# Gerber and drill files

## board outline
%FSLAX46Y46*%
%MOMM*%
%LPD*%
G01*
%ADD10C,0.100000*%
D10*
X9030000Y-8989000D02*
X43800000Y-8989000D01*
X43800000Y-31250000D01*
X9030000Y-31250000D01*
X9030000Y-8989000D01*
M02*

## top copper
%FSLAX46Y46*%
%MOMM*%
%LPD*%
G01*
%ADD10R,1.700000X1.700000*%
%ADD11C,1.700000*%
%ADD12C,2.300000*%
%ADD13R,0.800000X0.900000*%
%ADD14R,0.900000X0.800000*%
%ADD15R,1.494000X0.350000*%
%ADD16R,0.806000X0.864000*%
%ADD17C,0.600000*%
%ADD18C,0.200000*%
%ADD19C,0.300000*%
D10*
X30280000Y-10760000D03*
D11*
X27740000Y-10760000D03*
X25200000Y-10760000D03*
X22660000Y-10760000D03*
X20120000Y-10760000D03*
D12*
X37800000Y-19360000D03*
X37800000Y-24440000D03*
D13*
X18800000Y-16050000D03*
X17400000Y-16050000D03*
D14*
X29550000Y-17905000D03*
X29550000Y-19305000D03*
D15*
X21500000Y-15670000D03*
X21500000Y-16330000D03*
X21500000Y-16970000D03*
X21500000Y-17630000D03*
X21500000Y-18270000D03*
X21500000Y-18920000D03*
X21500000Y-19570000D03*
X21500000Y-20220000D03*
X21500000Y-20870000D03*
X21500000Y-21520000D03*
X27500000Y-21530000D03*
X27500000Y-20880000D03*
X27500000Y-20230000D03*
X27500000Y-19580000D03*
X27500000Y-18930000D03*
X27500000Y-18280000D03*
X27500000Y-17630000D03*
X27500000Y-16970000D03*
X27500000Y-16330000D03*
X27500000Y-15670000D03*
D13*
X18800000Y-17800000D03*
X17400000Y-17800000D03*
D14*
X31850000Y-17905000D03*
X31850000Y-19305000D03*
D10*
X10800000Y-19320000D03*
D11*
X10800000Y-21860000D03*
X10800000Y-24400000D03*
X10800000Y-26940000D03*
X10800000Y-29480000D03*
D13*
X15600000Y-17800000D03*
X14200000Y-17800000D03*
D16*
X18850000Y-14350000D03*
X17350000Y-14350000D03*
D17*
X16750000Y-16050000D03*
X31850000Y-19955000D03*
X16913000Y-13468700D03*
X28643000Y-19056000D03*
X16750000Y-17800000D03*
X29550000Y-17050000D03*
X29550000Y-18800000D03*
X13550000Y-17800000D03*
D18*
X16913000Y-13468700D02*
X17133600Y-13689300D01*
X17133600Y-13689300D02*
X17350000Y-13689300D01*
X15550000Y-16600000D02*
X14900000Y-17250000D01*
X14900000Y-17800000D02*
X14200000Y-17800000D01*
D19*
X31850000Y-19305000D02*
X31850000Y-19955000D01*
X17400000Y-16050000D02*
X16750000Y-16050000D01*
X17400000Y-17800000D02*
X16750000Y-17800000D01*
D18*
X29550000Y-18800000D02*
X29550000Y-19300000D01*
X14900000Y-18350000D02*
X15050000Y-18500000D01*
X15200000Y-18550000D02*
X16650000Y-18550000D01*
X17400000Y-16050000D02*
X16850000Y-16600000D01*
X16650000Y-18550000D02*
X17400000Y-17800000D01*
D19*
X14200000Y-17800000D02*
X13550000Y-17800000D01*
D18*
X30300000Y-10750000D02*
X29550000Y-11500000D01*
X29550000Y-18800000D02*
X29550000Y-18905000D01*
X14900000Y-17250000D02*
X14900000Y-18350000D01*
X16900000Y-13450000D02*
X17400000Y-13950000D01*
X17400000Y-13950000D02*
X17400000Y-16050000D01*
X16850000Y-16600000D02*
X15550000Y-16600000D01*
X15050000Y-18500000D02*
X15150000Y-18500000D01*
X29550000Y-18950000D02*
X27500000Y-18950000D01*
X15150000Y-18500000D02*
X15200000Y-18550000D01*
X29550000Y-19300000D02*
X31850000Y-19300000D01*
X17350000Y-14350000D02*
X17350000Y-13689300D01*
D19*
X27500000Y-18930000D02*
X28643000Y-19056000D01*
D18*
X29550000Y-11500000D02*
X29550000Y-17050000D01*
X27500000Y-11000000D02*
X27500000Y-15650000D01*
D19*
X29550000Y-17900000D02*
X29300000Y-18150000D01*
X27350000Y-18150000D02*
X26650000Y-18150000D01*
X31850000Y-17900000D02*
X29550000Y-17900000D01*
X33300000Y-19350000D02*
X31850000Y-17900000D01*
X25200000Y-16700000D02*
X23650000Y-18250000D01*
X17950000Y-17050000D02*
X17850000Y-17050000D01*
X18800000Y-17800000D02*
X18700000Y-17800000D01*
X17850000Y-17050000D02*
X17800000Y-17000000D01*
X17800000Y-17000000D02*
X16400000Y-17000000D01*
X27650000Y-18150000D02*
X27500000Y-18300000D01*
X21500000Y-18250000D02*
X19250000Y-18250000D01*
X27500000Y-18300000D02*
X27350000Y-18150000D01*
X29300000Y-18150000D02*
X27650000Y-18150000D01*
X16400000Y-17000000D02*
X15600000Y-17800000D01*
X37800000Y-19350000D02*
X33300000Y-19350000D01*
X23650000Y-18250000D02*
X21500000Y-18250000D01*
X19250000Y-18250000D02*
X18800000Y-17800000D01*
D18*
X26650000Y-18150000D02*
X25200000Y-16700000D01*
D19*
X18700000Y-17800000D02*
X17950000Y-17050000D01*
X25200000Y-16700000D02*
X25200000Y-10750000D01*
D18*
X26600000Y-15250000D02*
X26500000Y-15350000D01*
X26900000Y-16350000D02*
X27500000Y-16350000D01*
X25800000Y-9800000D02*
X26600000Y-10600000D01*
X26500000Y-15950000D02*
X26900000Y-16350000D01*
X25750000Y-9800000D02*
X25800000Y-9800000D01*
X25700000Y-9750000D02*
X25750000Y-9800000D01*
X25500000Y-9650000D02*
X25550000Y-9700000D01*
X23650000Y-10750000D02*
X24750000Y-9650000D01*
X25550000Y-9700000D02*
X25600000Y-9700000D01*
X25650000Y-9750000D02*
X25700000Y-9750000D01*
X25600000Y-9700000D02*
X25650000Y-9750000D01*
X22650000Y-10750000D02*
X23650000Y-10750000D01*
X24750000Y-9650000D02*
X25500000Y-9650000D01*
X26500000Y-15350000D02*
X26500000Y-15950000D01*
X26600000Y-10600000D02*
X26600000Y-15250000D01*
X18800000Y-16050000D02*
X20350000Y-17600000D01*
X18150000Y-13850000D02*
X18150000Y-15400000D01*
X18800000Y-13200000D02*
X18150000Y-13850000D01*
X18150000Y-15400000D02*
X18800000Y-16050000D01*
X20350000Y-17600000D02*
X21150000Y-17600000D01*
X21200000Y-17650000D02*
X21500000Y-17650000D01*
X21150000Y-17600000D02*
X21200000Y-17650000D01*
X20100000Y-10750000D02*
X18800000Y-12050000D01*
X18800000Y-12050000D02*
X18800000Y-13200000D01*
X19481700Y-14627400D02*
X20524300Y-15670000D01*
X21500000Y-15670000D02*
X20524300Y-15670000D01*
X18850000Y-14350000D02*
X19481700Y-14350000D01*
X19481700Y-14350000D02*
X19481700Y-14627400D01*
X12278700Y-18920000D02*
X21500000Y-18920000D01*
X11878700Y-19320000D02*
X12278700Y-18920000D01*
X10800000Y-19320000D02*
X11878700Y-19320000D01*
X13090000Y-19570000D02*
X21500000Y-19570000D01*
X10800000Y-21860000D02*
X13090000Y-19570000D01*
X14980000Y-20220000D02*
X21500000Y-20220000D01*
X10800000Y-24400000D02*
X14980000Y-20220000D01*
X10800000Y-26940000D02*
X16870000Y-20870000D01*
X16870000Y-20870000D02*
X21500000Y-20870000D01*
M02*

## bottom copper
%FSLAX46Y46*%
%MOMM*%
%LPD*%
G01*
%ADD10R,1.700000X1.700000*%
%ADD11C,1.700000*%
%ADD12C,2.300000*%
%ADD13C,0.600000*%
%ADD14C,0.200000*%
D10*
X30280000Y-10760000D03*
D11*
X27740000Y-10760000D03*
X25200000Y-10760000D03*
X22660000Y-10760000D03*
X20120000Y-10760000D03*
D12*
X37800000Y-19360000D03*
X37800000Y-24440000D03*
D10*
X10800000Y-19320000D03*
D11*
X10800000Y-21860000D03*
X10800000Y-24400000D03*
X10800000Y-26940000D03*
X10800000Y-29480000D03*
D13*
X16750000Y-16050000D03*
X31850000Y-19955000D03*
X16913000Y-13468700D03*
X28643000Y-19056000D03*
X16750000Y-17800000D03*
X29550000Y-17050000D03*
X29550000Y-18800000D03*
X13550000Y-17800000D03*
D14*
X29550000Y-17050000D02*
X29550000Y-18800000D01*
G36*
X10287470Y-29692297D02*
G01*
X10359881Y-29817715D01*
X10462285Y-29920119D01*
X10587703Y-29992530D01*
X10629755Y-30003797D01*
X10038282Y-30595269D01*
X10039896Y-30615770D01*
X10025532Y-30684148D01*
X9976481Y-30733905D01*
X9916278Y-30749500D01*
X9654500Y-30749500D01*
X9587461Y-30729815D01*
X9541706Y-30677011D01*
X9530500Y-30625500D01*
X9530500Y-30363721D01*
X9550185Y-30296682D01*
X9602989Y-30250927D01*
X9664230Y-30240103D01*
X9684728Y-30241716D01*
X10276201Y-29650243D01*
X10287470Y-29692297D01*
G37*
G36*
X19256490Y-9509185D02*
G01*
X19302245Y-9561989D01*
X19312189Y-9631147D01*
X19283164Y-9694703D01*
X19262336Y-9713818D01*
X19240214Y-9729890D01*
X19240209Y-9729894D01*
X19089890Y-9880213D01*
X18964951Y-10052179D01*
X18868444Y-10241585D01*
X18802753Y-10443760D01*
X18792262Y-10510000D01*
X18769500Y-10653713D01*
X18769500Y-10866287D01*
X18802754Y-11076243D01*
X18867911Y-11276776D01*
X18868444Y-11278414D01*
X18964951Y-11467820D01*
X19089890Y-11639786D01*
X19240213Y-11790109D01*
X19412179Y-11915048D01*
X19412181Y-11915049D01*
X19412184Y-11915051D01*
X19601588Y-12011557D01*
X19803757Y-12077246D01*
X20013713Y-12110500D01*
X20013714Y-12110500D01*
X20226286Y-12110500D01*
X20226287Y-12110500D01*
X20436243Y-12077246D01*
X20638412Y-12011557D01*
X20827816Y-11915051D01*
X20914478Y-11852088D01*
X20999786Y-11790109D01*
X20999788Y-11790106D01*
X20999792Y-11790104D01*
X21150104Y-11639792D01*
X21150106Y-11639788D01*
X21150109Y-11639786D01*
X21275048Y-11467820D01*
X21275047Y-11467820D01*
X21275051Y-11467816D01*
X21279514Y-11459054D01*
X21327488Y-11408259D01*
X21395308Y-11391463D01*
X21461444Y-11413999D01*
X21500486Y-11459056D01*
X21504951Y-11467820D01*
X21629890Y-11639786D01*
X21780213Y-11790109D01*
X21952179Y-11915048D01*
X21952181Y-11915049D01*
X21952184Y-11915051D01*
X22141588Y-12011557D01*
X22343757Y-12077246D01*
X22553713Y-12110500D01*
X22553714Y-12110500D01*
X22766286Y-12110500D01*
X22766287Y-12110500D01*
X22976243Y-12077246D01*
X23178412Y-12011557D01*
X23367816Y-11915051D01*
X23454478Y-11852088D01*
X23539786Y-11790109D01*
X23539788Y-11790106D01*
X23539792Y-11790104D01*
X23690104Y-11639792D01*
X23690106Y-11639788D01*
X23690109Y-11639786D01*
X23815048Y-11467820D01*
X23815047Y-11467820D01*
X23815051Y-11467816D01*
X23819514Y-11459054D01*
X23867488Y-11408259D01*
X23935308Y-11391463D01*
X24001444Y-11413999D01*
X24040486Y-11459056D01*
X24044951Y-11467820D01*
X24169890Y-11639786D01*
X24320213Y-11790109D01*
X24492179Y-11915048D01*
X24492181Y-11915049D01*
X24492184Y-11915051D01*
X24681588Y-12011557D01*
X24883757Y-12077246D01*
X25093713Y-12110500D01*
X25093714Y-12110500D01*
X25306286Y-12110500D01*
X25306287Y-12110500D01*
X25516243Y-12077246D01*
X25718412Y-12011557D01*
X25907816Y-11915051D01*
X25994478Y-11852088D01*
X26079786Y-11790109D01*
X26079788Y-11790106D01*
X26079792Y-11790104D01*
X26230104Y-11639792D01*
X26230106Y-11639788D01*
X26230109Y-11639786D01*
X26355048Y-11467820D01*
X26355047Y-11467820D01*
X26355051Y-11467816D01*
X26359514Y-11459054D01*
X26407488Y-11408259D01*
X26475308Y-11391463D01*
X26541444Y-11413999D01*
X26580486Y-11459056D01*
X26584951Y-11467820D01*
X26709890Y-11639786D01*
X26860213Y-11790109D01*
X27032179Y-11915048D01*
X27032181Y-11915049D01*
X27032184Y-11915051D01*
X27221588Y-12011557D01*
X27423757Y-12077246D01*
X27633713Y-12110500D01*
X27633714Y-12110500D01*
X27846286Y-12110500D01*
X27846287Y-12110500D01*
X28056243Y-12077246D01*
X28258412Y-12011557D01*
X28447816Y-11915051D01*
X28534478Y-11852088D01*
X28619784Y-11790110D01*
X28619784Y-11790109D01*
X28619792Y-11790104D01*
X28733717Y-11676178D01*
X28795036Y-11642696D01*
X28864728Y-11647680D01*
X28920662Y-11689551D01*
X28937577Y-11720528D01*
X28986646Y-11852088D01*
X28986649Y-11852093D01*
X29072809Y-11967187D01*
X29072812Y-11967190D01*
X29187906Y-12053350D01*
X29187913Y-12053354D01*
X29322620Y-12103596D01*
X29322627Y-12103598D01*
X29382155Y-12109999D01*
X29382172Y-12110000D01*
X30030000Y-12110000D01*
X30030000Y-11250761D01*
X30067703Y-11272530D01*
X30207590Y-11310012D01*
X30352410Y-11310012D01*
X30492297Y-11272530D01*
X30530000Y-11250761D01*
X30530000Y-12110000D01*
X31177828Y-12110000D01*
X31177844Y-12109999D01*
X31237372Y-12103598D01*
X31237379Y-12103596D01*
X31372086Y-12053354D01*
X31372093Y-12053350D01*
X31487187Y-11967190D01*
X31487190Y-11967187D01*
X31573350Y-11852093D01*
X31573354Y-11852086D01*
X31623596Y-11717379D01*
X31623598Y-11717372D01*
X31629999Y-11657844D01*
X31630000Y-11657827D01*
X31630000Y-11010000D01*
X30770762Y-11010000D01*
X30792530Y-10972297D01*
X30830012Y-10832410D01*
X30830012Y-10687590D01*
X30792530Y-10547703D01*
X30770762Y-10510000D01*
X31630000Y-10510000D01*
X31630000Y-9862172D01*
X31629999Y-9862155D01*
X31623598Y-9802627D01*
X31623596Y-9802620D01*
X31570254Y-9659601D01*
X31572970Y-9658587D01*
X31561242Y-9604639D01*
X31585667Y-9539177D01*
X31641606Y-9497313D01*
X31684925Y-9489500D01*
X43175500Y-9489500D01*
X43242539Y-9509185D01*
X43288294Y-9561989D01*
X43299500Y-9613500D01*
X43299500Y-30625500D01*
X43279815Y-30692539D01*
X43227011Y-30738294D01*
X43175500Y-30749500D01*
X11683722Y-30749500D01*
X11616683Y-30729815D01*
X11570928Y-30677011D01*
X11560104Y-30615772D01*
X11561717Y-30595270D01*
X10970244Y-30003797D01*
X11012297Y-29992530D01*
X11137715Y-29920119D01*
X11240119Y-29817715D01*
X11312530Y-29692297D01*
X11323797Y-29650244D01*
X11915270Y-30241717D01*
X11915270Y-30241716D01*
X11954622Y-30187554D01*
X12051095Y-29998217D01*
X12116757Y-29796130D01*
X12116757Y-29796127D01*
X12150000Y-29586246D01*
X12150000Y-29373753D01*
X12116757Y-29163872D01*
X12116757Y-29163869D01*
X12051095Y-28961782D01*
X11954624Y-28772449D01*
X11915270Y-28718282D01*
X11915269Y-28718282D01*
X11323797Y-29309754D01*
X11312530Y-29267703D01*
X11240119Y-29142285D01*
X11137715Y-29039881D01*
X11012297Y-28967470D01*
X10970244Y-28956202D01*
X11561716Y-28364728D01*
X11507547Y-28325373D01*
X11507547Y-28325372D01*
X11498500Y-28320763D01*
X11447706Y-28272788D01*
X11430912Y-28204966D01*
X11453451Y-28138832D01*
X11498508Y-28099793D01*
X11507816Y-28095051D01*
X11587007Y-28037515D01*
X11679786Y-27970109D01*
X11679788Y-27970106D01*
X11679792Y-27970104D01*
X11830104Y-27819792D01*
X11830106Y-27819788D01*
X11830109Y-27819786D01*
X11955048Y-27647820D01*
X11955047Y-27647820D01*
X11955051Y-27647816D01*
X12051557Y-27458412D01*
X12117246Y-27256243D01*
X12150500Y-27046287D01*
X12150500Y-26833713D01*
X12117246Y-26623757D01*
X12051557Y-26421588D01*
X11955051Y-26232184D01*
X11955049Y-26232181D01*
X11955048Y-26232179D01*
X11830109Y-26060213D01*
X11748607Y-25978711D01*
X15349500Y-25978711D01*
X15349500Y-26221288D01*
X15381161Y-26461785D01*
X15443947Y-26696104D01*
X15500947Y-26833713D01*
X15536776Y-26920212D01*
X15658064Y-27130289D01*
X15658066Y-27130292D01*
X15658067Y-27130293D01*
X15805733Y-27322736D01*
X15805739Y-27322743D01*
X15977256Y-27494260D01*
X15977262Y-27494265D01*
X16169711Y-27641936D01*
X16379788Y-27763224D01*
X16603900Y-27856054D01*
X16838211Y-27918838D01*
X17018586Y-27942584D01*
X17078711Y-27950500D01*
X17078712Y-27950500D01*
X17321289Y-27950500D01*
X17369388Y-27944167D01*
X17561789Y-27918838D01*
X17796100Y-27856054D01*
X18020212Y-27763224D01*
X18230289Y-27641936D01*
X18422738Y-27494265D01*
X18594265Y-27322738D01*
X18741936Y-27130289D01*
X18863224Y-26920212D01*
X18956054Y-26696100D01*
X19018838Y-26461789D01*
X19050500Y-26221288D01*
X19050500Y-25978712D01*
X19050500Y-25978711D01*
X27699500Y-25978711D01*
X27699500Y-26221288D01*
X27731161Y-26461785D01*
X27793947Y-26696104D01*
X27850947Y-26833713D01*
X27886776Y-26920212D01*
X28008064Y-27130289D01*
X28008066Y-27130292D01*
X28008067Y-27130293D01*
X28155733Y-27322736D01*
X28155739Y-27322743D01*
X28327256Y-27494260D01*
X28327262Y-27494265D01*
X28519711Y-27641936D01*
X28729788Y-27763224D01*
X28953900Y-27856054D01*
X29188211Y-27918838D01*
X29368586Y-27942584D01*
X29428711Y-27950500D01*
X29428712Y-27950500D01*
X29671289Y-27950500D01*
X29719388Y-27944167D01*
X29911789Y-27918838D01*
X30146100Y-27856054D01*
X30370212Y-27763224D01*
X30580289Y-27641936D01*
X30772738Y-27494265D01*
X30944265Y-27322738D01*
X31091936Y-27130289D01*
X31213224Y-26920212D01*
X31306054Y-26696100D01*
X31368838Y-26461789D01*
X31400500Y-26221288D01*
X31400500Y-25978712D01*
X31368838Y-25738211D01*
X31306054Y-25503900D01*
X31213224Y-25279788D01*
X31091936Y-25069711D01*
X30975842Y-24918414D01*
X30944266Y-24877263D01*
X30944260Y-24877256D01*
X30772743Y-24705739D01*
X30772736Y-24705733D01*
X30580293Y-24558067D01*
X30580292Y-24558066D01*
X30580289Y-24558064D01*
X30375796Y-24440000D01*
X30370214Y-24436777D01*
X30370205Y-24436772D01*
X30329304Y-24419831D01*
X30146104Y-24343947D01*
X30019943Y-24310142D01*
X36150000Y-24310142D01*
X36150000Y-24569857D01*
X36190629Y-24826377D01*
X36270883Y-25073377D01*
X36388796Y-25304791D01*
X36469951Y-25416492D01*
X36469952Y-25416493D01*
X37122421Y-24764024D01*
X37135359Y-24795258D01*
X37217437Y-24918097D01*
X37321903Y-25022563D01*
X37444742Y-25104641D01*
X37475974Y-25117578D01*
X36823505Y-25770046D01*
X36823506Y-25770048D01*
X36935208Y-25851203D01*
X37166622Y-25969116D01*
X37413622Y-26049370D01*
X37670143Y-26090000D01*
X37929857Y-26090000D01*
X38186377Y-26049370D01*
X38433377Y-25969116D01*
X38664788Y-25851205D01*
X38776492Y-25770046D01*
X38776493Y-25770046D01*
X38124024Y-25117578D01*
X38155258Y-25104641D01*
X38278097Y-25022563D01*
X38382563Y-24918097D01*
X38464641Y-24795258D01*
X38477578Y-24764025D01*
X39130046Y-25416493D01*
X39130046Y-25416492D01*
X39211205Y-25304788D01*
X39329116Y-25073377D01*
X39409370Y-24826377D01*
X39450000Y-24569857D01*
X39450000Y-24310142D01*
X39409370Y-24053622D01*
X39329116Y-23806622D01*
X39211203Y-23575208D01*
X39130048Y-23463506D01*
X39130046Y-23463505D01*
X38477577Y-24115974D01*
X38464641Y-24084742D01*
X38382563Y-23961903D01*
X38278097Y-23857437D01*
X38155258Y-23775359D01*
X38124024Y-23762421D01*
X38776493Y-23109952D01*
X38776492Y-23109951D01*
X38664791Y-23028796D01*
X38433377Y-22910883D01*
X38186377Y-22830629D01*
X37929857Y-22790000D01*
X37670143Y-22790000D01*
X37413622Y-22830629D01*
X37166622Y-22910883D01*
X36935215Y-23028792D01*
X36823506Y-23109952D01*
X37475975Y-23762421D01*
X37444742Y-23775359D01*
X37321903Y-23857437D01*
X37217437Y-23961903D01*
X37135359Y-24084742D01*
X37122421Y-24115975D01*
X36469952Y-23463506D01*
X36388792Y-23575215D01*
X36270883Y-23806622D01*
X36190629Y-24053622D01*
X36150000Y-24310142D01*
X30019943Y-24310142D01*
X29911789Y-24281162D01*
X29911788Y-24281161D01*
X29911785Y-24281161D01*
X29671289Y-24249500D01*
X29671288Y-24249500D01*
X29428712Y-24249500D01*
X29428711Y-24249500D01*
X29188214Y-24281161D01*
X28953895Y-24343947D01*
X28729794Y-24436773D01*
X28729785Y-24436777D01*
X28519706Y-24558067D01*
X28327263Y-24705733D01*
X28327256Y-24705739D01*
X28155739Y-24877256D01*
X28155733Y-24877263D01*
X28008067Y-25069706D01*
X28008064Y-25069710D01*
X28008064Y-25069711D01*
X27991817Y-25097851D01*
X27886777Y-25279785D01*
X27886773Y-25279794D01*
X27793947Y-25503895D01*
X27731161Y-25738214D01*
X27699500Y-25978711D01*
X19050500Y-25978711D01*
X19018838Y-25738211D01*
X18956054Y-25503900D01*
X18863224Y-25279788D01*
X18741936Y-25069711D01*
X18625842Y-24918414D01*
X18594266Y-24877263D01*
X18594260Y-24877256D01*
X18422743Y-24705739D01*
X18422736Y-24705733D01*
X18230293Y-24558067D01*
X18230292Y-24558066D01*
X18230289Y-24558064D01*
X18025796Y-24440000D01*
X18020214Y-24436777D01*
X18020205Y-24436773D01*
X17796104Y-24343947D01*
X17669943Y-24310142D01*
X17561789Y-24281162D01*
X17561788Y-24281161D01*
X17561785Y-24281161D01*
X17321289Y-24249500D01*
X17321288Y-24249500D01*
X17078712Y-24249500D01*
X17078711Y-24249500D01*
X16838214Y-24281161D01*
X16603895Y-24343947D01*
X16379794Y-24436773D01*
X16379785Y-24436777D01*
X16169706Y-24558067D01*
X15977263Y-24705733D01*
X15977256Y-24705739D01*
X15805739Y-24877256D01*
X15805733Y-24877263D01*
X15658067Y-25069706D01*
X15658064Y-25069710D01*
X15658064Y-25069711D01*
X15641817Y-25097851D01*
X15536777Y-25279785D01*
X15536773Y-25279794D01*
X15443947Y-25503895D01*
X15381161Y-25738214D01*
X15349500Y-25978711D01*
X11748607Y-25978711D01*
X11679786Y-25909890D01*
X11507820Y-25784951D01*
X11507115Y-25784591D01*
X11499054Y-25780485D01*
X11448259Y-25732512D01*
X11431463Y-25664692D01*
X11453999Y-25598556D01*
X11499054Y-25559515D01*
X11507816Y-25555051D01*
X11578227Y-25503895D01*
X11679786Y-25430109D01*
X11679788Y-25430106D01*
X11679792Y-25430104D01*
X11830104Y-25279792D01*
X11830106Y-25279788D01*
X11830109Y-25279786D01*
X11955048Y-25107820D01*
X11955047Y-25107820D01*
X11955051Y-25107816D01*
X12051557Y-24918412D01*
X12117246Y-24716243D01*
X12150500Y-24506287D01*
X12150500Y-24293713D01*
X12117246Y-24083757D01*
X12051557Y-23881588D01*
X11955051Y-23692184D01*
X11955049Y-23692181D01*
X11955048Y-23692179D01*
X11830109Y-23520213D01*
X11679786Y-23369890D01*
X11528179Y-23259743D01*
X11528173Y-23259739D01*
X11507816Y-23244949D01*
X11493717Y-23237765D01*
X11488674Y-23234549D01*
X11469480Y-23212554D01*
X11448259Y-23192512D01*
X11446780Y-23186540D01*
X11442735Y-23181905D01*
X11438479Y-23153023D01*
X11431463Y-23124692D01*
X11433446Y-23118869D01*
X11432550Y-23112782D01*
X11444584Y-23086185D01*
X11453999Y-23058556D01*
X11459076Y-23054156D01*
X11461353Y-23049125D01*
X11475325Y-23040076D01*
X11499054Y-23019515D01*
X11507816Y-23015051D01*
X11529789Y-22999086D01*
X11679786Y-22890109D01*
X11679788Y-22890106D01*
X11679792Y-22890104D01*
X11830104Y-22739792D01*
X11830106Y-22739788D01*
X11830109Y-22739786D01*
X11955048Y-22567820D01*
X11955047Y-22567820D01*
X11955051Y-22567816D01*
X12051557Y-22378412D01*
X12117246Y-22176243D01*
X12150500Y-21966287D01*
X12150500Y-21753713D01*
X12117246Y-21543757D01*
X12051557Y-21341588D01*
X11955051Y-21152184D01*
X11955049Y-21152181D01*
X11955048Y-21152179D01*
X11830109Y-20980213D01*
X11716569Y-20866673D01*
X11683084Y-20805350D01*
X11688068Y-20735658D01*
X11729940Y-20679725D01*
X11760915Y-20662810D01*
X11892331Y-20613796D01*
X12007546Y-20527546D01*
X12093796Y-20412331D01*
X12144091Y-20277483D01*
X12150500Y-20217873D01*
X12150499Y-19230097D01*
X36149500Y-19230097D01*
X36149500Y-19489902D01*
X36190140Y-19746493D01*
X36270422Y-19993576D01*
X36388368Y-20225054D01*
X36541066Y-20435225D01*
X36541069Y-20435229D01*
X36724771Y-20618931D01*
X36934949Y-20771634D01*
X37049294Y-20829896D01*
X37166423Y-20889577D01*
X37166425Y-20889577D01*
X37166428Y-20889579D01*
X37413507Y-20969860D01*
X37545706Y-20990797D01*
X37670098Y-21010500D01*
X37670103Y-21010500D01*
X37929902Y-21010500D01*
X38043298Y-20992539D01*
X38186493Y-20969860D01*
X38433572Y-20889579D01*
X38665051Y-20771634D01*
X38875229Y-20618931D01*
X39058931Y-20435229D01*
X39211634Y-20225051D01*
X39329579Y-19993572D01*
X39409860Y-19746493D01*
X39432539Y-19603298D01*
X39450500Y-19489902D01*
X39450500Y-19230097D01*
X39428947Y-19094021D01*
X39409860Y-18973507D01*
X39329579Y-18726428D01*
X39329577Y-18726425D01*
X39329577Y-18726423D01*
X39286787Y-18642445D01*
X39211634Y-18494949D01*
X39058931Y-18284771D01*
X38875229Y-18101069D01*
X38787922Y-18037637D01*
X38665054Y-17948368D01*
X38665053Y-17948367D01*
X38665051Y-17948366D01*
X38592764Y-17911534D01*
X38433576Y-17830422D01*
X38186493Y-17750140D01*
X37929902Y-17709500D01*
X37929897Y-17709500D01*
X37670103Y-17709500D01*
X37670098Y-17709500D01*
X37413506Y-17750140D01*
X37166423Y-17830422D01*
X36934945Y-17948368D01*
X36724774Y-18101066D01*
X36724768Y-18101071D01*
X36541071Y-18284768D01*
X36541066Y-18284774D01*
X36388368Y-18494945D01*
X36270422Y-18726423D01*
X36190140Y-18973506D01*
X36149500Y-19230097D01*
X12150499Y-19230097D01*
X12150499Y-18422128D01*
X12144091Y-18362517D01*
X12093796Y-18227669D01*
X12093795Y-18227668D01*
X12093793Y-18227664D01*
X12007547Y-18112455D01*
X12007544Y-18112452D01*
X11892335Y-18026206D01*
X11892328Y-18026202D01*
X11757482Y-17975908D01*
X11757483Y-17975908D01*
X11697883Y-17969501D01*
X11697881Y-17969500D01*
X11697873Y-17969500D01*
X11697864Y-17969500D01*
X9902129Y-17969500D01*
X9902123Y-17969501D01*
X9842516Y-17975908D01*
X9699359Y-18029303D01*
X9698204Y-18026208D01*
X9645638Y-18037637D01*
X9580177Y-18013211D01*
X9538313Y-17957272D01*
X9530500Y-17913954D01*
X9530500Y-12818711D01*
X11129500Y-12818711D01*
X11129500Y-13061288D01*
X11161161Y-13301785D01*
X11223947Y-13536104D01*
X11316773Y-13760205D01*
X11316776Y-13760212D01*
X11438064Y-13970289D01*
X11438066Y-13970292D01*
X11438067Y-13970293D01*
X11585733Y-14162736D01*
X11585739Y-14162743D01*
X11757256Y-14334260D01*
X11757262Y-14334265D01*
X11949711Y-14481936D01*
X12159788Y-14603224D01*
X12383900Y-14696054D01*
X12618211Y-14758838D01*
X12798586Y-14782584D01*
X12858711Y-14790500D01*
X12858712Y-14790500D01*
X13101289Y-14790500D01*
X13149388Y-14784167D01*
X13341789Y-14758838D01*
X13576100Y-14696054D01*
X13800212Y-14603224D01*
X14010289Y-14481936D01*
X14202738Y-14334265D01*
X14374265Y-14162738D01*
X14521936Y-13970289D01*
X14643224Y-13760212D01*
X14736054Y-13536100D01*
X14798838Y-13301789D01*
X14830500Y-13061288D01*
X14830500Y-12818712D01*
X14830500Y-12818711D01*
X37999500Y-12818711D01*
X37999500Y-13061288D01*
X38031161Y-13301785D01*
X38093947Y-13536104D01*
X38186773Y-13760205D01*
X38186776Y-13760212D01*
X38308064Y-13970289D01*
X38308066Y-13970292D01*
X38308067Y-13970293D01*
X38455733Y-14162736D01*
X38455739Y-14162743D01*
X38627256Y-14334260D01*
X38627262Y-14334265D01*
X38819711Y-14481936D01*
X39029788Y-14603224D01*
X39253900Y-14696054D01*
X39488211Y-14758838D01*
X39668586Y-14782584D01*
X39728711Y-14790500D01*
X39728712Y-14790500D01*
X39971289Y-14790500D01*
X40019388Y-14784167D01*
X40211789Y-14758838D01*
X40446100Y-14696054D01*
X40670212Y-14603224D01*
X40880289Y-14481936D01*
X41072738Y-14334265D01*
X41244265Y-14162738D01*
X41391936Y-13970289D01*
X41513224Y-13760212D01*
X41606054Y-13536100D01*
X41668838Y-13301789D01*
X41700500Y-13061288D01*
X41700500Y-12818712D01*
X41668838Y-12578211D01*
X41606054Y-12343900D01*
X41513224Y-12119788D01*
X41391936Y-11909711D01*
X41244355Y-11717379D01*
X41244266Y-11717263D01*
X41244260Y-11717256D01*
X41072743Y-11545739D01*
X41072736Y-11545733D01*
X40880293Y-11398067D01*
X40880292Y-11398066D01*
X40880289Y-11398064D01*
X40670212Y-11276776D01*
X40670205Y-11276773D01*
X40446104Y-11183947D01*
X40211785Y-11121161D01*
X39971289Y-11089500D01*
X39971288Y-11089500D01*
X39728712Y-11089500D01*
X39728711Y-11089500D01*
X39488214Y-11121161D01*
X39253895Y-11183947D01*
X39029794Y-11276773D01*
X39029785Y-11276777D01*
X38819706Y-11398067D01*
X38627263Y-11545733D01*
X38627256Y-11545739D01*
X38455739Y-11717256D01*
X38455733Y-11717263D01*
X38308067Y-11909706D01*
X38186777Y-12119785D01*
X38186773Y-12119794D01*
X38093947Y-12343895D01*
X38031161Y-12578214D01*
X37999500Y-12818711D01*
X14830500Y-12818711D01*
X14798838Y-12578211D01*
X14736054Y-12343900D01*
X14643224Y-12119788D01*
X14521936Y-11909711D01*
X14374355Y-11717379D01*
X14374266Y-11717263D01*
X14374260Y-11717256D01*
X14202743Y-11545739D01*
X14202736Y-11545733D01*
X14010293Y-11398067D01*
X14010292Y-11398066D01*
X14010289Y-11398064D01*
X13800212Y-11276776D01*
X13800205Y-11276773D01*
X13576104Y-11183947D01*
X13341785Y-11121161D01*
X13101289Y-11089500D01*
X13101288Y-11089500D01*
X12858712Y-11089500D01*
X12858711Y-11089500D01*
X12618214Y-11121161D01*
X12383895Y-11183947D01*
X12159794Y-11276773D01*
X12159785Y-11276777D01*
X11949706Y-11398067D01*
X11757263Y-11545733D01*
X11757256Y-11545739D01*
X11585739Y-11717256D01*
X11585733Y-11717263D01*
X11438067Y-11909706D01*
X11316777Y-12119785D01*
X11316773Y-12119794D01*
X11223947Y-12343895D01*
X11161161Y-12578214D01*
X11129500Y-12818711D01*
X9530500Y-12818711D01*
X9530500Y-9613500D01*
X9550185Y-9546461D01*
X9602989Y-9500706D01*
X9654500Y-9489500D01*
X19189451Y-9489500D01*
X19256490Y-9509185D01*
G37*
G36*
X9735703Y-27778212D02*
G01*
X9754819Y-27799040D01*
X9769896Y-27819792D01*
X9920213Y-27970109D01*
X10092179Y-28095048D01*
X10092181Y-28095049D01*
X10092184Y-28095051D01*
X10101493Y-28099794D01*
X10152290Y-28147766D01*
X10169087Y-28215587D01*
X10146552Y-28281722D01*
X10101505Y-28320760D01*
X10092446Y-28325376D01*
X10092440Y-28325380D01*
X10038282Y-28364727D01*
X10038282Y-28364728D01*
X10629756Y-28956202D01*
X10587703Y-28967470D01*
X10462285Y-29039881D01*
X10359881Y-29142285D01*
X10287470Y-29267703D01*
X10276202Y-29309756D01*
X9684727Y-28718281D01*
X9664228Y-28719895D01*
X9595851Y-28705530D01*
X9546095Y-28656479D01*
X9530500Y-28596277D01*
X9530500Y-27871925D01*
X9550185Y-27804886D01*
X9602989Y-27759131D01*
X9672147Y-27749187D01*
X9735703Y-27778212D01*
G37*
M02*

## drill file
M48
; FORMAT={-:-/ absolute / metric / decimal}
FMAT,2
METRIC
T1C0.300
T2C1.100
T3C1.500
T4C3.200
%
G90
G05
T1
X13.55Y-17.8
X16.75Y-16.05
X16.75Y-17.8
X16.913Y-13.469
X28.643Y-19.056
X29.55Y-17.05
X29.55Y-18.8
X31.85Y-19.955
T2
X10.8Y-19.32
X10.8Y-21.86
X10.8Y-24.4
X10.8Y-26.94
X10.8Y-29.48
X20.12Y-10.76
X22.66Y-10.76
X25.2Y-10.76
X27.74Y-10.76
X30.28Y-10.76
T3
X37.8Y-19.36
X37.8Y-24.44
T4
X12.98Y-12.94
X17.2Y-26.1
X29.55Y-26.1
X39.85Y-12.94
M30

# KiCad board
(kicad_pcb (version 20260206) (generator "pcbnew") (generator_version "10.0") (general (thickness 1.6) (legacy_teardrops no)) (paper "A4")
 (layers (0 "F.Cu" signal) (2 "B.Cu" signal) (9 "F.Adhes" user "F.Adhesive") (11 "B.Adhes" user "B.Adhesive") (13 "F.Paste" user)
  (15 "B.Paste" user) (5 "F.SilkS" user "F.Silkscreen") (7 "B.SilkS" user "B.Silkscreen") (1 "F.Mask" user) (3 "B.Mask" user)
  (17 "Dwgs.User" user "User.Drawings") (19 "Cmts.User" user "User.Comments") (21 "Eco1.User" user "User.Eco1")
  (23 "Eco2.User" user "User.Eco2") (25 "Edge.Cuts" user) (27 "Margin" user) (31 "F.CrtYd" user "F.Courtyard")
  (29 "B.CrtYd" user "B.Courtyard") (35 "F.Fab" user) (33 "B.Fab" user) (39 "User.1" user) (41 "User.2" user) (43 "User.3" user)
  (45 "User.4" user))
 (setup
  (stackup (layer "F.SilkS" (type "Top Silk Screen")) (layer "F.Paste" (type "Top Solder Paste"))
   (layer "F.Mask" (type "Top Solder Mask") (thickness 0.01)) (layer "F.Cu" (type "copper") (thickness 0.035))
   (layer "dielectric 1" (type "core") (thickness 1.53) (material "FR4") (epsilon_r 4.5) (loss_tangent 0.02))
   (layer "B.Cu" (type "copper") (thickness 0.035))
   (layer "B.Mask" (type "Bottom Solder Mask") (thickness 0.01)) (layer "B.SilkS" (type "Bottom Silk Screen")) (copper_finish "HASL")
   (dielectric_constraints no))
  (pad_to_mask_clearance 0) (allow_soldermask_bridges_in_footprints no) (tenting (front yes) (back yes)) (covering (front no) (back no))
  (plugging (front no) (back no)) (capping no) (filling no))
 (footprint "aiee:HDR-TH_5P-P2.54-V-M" (layer "F.Cu") (at 25.2 10.76 180)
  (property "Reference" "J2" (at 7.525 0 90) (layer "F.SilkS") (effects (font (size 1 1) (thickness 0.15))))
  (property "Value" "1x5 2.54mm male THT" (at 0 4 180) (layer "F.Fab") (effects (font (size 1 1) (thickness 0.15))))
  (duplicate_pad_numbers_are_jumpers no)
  (pad "1" thru_hole rect (at -5.08 0 180) (size 1.7 1.7) (drill 1.100024) (layers "*.Cu" "*.Mask") (remove_unused_layers no) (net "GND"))
  (pad "2" thru_hole circle (at -2.54 0 180) (size 1.7 1.7) (drill 1.100024) (layers "*.Cu" "*.Mask") (remove_unused_layers no)
   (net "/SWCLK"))
  (pad "3" thru_hole circle (at 0 0 180) (size 1.7 1.7) (drill 1.100024) (layers "*.Cu" "*.Mask") (remove_unused_layers no) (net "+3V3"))
  (pad "4" thru_hole circle (at 2.54 0 180) (size 1.7 1.7) (drill 1.100024) (layers "*.Cu" "*.Mask") (remove_unused_layers no)
   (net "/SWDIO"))
  (pad "5" thru_hole circle (at 5.08 0 180) (size 1.7 1.7) (drill 1.100024) (layers "*.Cu" "*.Mask") (remove_unused_layers no) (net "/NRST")))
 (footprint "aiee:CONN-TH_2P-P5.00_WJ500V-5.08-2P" (layer "F.Cu") (at 37.8 21.9 -90)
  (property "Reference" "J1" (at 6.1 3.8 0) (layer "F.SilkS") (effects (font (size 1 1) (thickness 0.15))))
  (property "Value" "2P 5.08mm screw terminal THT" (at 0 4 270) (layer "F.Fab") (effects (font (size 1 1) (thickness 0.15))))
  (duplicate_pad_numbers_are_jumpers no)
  (pad "1" thru_hole circle (at -2.54 0 90) (size 2.3 2.3) (drill 1.5) (layers "*.Cu" "*.Mask") (remove_unused_layers no) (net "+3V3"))
  (pad "2" thru_hole circle (at 2.54 0 90) (size 2.3 2.3) (drill 1.5) (layers "*.Cu" "*.Mask") (remove_unused_layers no) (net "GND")))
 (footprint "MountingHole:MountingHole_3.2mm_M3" (layer "F.Cu") (at 29.55 26.1)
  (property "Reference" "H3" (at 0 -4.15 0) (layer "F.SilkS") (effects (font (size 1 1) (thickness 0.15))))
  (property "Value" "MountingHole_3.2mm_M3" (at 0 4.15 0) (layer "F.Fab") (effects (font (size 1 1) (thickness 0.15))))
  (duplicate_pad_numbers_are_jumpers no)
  (pad "" np_thru_hole circle (at 0 0) (size 3.2 3.2) (drill 3.2) (layers "*.Cu" "*.Mask")))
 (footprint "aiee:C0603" (layer "F.Cu") (at 18.1 16.05 180)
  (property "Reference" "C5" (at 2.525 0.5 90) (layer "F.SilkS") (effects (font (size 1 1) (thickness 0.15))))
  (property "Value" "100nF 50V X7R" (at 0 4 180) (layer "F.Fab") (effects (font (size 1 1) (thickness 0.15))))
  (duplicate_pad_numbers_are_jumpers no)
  (pad "1" smd rect (at -0.7 0 180) (size 0.8 0.9) (layers "F.Cu" "F.Mask" "F.Paste") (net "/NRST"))
  (pad "2" smd rect (at 0.7 0 180) (size 0.8 0.9) (layers "F.Cu" "F.Mask" "F.Paste") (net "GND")))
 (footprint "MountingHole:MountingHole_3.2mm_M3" (layer "F.Cu") (at 17.2 26.1)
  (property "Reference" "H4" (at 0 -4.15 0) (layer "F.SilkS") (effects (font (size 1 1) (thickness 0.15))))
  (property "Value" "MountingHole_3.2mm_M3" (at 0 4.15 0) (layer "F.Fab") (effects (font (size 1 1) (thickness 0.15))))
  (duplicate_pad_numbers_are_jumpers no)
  (pad "" np_thru_hole circle (at 0 0) (size 3.2 3.2) (drill 3.2) (layers "*.Cu" "*.Mask")))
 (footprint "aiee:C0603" (layer "F.Cu") (at 29.55 18.605 -90)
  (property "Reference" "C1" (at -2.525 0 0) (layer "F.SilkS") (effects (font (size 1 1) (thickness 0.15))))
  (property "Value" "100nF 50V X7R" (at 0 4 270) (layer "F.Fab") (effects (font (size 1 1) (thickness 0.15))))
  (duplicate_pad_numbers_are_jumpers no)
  (pad "1" smd rect (at -0.7 0 270) (size 0.8 0.9) (layers "F.Cu" "F.Mask" "F.Paste") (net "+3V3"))
  (pad "2" smd rect (at 0.7 0 270) (size 0.8 0.9) (layers "F.Cu" "F.Mask" "F.Paste") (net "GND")))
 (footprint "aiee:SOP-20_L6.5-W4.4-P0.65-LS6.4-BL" (layer "F.Cu") (at 24.5 18.6 -90)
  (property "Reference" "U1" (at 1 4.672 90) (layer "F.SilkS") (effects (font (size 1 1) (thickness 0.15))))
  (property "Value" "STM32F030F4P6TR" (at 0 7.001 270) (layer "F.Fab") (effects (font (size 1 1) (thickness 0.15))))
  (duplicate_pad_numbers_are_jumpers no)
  (pad "1" smd rect (at -2.93 3 270) (size 0.35 1.494) (layers "F.Cu" "F.Mask" "F.Paste") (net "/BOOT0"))
  (pad "2" smd rect (at -2.27 3 270) (size 0.35 1.494) (layers "F.Cu" "F.Mask" "F.Paste") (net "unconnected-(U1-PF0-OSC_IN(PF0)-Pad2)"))
  (pad "3" smd rect (at -1.63 3 270) (size 0.35 1.494) (layers "F.Cu" "F.Mask" "F.Paste") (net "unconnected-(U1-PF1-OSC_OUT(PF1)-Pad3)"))
  (pad "4" smd rect (at -0.97 3 270) (size 0.35 1.494) (layers "F.Cu" "F.Mask" "F.Paste") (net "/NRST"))
  (pad "5" smd rect (at -0.33 3 270) (size 0.35 1.494) (layers "F.Cu" "F.Mask" "F.Paste") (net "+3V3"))
  (pad "6" smd rect (at 0.32 3 270) (size 0.35 1.494) (layers "F.Cu" "F.Mask" "F.Paste") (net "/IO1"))
  (pad "7" smd rect (at 0.97 3 270) (size 0.35 1.494) (layers "F.Cu" "F.Mask" "F.Paste") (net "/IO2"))
  (pad "8" smd rect (at 1.62 3 270) (size 0.35 1.494) (layers "F.Cu" "F.Mask" "F.Paste") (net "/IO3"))
  (pad "9" smd rect (at 2.27 3 270) (size 0.35 1.494) (layers "F.Cu" "F.Mask" "F.Paste") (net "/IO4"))
  (pad "10" smd rect (at 2.92 3 270) (size 0.35 1.494) (layers "F.Cu" "F.Mask" "F.Paste") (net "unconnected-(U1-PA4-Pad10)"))
  (pad "11" smd rect (at 2.93 -3 270) (size 0.35 1.494) (layers "F.Cu" "F.Mask" "F.Paste") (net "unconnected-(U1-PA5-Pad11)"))
  (pad "12" smd rect (at 2.28 -3 270) (size 0.35 1.494) (layers "F.Cu" "F.Mask" "F.Paste") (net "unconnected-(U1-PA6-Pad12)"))
  (pad "13" smd rect (at 1.63 -3 270) (size 0.35 1.494) (layers "F.Cu" "F.Mask" "F.Paste") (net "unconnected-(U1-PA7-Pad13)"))
  (pad "14" smd rect (at 0.98 -3 270) (size 0.35 1.494) (layers "F.Cu" "F.Mask" "F.Paste") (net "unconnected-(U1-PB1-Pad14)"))
  (pad "15" smd rect (at 0.33 -3 270) (size 0.35 1.494) (layers "F.Cu" "F.Mask" "F.Paste") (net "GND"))
  (pad "16" smd rect (at -0.32 -3 270) (size 0.35 1.494) (layers "F.Cu" "F.Mask" "F.Paste") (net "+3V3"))
  (pad "17" smd rect (at -0.97 -3 270) (size 0.35 1.494) (layers "F.Cu" "F.Mask" "F.Paste") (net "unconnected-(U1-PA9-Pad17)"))
  (pad "18" smd rect (at -1.63 -3 270) (size 0.35 1.494) (layers "F.Cu" "F.Mask" "F.Paste") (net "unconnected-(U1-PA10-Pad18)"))
  (pad "19" smd rect (at -2.27 -3 270) (size 0.35 1.494) (layers "F.Cu" "F.Mask" "F.Paste") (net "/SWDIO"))
  (pad "20" smd rect (at -2.93 -3 270) (size 0.35 1.494) (layers "F.Cu" "F.Mask" "F.Paste") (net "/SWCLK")))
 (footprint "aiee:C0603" (layer "F.Cu") (at 18.1 17.8 180)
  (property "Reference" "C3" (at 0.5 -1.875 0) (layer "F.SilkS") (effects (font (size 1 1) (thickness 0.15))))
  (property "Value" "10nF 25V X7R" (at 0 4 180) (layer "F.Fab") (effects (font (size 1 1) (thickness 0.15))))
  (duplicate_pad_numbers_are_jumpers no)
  (pad "1" smd rect (at -0.7 0 180) (size 0.8 0.9) (layers "F.Cu" "F.Mask" "F.Paste") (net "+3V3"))
  (pad "2" smd rect (at 0.7 0 180) (size 0.8 0.9) (layers "F.Cu" "F.Mask" "F.Paste") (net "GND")))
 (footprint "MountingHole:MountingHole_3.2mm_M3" (layer "F.Cu") (at 12.98 12.94)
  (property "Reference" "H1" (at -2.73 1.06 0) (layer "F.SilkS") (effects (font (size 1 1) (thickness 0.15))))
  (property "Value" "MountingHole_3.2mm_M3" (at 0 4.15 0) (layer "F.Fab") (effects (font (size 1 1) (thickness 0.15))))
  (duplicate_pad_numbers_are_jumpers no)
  (pad "" np_thru_hole circle (at 0 0) (size 3.2 3.2) (drill 3.2) (layers "*.Cu" "*.Mask")))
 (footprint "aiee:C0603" (layer "F.Cu") (at 31.85 18.605 -90)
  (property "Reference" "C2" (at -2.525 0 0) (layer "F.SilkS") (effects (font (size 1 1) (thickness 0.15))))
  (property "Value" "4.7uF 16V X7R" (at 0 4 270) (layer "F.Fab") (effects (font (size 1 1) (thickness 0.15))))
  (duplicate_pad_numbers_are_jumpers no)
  (pad "1" smd rect (at -0.7 0 270) (size 0.8 0.9) (layers "F.Cu" "F.Mask" "F.Paste") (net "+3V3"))
  (pad "2" smd rect (at 0.7 0 270) (size 0.8 0.9) (layers "F.Cu" "F.Mask" "F.Paste") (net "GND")))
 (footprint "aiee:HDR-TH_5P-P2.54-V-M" (layer "F.Cu") (at 10.8 24.4 -90)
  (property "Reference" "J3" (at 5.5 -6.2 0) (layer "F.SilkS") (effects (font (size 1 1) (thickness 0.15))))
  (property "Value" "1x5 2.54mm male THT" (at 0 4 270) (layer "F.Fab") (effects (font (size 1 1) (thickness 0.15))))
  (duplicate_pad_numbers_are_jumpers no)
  (pad "1" thru_hole rect (at -5.08 0 270) (size 1.7 1.7) (drill 1.100024) (layers "*.Cu" "*.Mask") (remove_unused_layers no) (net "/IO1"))
  (pad "2" thru_hole circle (at -2.54 0 270) (size 1.7 1.7) (drill 1.100024) (layers "*.Cu" "*.Mask") (remove_unused_layers no) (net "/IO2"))
  (pad "3" thru_hole circle (at 0 0 270) (size 1.7 1.7) (drill 1.100024) (layers "*.Cu" "*.Mask") (remove_unused_layers no) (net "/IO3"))
  (pad "4" thru_hole circle (at 2.54 0 270) (size 1.7 1.7) (drill 1.100024) (layers "*.Cu" "*.Mask") (remove_unused_layers no) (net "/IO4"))
  (pad "5" thru_hole circle (at 5.08 0 270) (size 1.7 1.7) (drill 1.100024) (layers "*.Cu" "*.Mask") (remove_unused_layers no) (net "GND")))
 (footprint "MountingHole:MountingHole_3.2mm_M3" (layer "F.Cu") (at 39.85 12.94)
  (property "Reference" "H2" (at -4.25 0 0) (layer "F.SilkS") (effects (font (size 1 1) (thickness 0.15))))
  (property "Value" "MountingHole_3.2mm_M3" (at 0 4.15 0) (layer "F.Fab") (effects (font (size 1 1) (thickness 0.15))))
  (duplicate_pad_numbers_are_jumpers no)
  (pad "" np_thru_hole circle (at 0 0) (size 3.2 3.2) (drill 3.2) (layers "*.Cu" "*.Mask")))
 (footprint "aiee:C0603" (layer "F.Cu") (at 14.9 17.8 180)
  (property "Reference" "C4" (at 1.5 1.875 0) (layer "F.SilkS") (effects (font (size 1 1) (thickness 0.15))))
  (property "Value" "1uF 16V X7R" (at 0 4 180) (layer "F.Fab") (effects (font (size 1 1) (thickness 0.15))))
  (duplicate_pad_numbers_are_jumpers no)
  (pad "1" smd rect (at -0.7 0 180) (size 0.8 0.9) (layers "F.Cu" "F.Mask" "F.Paste") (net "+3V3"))
  (pad "2" smd rect (at 0.7 0 180) (size 0.8 0.9) (layers "F.Cu" "F.Mask" "F.Paste") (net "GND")))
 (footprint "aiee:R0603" (layer "F.Cu") (at 18.1 14.35 180)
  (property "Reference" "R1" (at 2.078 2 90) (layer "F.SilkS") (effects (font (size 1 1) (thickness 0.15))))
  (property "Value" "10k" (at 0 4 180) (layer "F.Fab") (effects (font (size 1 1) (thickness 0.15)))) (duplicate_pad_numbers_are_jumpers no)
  (pad "1" smd rect (at -0.75 0 180) (size 0.806 0.864) (layers "F.Cu" "F.Mask" "F.Paste") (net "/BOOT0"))
  (pad "2" smd rect (at 0.75 0 180) (size 0.806 0.864) (layers "F.Cu" "F.Mask" "F.Paste") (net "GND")))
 (gr_rect (start 9.03 8.989) (end 43.8 31.25) (stroke (width 0.1) (type default)) (fill no) (layer "Edge.Cuts"))
 (segment (start 16.913 13.4687) (end 17.1336 13.6893) (width 0.2) (layer "F.Cu") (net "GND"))
 (segment (start 17.1336 13.6893) (end 17.35 13.6893) (width 0.2) (layer "F.Cu") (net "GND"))
 (segment (start 15.55 16.6) (end 14.9 17.25) (width 0.2) (layer "F.Cu") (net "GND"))
 (segment (start 14.9 17.8) (end 14.2 17.8) (width 0.2) (layer "F.Cu") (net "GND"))
 (segment (start 31.85 19.305) (end 31.85 19.955) (width 0.3) (layer "F.Cu") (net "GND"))
 (segment (start 17.4 16.05) (end 16.75 16.05) (width 0.3) (layer "F.Cu") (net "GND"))
 (segment (start 17.4 17.8) (end 16.75 17.8) (width 0.3) (layer "F.Cu") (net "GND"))
 (segment (start 29.55 18.8) (end 29.55 19.3) (width 0.2) (layer "F.Cu") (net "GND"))
 (segment (start 14.9 18.35) (end 15.05 18.5) (width 0.2) (layer "F.Cu") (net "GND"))
 (segment (start 15.2 18.55) (end 16.65 18.55) (width 0.2) (layer "F.Cu") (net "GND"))
 (segment (start 17.4 16.05) (end 16.85 16.6) (width 0.2) (layer "F.Cu") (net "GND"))
 (segment (start 16.65 18.55) (end 17.4 17.8) (width 0.2) (layer "F.Cu") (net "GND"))
 (segment (start 14.2 17.8) (end 13.55 17.8) (width 0.3) (layer "F.Cu") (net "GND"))
 (segment (start 30.3 10.75) (end 29.55 11.5) (width 0.2) (layer "F.Cu") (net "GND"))
 (segment (start 29.55 18.8) (end 29.55 18.905) (width 0.2) (layer "F.Cu") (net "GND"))
 (segment (start 14.9 17.25) (end 14.9 18.35) (width 0.2) (layer "F.Cu") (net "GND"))
 (segment (start 16.9 13.45) (end 17.4 13.95) (width 0.2) (layer "F.Cu") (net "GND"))
 (segment (start 17.4 13.95) (end 17.4 16.05) (width 0.2) (layer "F.Cu") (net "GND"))
 (segment (start 16.85 16.6) (end 15.55 16.6) (width 0.2) (layer "F.Cu") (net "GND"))
 (segment (start 15.05 18.5) (end 15.15 18.5) (width 0.2) (layer "F.Cu") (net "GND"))
 (segment (start 29.55 18.95) (end 27.5 18.95) (width 0.2) (layer "F.Cu") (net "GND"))
 (segment (start 15.15 18.5) (end 15.2 18.55) (width 0.2) (layer "F.Cu") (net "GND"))
 (segment (start 29.55 19.3) (end 31.85 19.3) (width 0.2) (layer "F.Cu") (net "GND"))
 (segment (start 17.35 14.35) (end 17.35 13.6893) (width 0.2) (layer "F.Cu") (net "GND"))
 (segment (start 27.5 18.93) (end 28.643 19.056) (width 0.3) (layer "F.Cu") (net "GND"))
 (segment (start 29.55 11.5) (end 29.55 17.05) (width 0.2) (layer "F.Cu") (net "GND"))
 (via (at 16.75 16.05) (size 0.6) (drill 0.3) (layers "F.Cu" "B.Cu") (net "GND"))
 (via (at 31.85 19.955) (size 0.6) (drill 0.3) (layers "F.Cu" "B.Cu") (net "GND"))
 (via (at 16.913 13.4687) (size 0.6) (drill 0.3) (layers "F.Cu" "B.Cu") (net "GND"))
 (via (at 28.643 19.056) (size 0.6) (drill 0.3) (layers "F.Cu" "B.Cu") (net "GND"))
 (via (at 16.75 17.8) (size 0.6) (drill 0.3) (layers "F.Cu" "B.Cu") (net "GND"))
 (via (at 29.55 17.05) (size 0.6) (drill 0.3) (layers "F.Cu" "B.Cu") (tenting (front yes) (back yes)) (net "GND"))
 (via (at 29.55 18.8) (size 0.6) (drill 0.3) (layers "F.Cu" "B.Cu") (tenting (front yes) (back yes)) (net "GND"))
 (via (at 13.55 17.8) (size 0.6) (drill 0.3) (layers "F.Cu" "B.Cu") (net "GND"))
 (segment (start 29.55 17.05) (end 29.55 18.8) (width 0.2) (layer "B.Cu") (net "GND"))
 (segment (start 27.5 11) (end 27.5 15.65) (width 0.2) (layer "F.Cu") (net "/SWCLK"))
 (segment (start 29.55 17.9) (end 29.3 18.15) (width 0.3) (layer "F.Cu") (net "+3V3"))
 (segment (start 27.35 18.15) (end 26.65 18.15) (width 0.3) (layer "F.Cu") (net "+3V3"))
 (segment (start 31.85 17.9) (end 29.55 17.9) (width 0.3) (layer "F.Cu") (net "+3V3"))
 (segment (start 33.3 19.35) (end 31.85 17.9) (width 0.3) (layer "F.Cu") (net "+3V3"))
 (segment (start 25.2 16.7) (end 23.65 18.25) (width 0.3) (layer "F.Cu") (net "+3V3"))
 (segment (start 17.95 17.05) (end 17.85 17.05) (width 0.3) (layer "F.Cu") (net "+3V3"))
 (segment (start 18.8 17.8) (end 18.7 17.8) (width 0.3) (layer "F.Cu") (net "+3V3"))
 (segment (start 17.85 17.05) (end 17.8 17) (width 0.3) (layer "F.Cu") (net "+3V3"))
 (segment (start 17.8 17) (end 16.4 17) (width 0.3) (layer "F.Cu") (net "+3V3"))
 (segment (start 27.65 18.15) (end 27.5 18.3) (width 0.3) (layer "F.Cu") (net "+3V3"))
 (segment (start 21.5 18.25) (end 19.25 18.25) (width 0.3) (layer "F.Cu") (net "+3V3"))
 (segment (start 27.5 18.3) (end 27.35 18.15) (width 0.3) (layer "F.Cu") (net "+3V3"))
 (segment (start 29.3 18.15) (end 27.65 18.15) (width 0.3) (layer "F.Cu") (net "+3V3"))
 (segment (start 16.4 17) (end 15.6 17.8) (width 0.3) (layer "F.Cu") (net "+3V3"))
 (segment (start 37.8 19.35) (end 33.3 19.35) (width 0.3) (layer "F.Cu") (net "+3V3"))
 (segment (start 23.65 18.25) (end 21.5 18.25) (width 0.3) (layer "F.Cu") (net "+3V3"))
 (segment (start 19.25 18.25) (end 18.8 17.8) (width 0.3) (layer "F.Cu") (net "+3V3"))
 (segment (start 26.65 18.15) (end 25.2 16.7) (width 0.2) (layer "F.Cu") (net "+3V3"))
 (segment (start 18.7 17.8) (end 17.95 17.05) (width 0.3) (layer "F.Cu") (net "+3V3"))
 (segment (start 25.2 16.7) (end 25.2 10.75) (width 0.3) (layer "F.Cu") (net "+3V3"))
 (segment (start 26.6 15.25) (end 26.5 15.35) (width 0.2) (layer "F.Cu") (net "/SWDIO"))
 (segment (start 26.9 16.35) (end 27.5 16.35) (width 0.2) (layer "F.Cu") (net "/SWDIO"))
 (segment (start 25.8 9.8) (end 26.6 10.6) (width 0.2) (layer "F.Cu") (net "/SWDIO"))
 (segment (start 26.5 15.95) (end 26.9 16.35) (width 0.2) (layer "F.Cu") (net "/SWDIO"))
 (segment (start 25.75 9.8) (end 25.8 9.8) (width 0.2) (layer "F.Cu") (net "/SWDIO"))
 (segment (start 25.7 9.75) (end 25.75 9.8) (width 0.2) (layer "F.Cu") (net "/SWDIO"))
 (segment (start 25.5 9.65) (end 25.55 9.7) (width 0.2) (layer "F.Cu") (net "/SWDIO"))
 (segment (start 23.65 10.75) (end 24.75 9.65) (width 0.2) (layer "F.Cu") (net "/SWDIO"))
 (segment (start 25.55 9.7) (end 25.6 9.7) (width 0.2) (layer "F.Cu") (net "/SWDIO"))
 (segment (start 25.65 9.75) (end 25.7 9.75) (width 0.2) (layer "F.Cu") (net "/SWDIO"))
 (segment (start 25.6 9.7) (end 25.65 9.75) (width 0.2) (layer "F.Cu") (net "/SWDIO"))
 (segment (start 22.65 10.75) (end 23.65 10.75) (width 0.2) (layer "F.Cu") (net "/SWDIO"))
 (segment (start 24.75 9.65) (end 25.5 9.65) (width 0.2) (layer "F.Cu") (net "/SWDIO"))
 (segment (start 26.5 15.35) (end 26.5 15.95) (width 0.2) (layer "F.Cu") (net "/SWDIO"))
 (segment (start 26.6 10.6) (end 26.6 15.25) (width 0.2) (layer "F.Cu") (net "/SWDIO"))
 (segment (start 18.8 16.05) (end 20.35 17.6) (width 0.2) (layer "F.Cu") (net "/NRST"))
 (segment (start 18.15 13.85) (end 18.15 15.4) (width 0.2) (layer "F.Cu") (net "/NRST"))
 (segment (start 18.8 13.2) (end 18.15 13.85) (width 0.2) (layer "F.Cu") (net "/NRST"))
 (segment (start 18.15 15.4) (end 18.8 16.05) (width 0.2) (layer "F.Cu") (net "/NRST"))
 (segment (start 20.35 17.6) (end 21.15 17.6) (width 0.2) (layer "F.Cu") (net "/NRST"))
 (segment (start 21.2 17.65) (end 21.5 17.65) (width 0.2) (layer "F.Cu") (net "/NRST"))
 (segment (start 21.15 17.6) (end 21.2 17.65) (width 0.2) (layer "F.Cu") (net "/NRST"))
 (segment (start 20.1 10.75) (end 18.8 12.05) (width 0.2) (layer "F.Cu") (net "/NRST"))
 (segment (start 18.8 12.05) (end 18.8 13.2) (width 0.2) (layer "F.Cu") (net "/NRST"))
 (segment (start 19.4817 14.6274) (end 20.5243 15.67) (width 0.2) (layer "F.Cu") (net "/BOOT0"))
 (segment (start 21.5 15.67) (end 20.5243 15.67) (width 0.2) (layer "F.Cu") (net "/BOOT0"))
 (segment (start 18.85 14.35) (end 19.4817 14.35) (width 0.2) (layer "F.Cu") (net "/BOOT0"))
 (segment (start 19.4817 14.35) (end 19.4817 14.6274) (width 0.2) (layer "F.Cu") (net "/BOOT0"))
 (segment (start 12.2787 18.92) (end 21.5 18.92) (width 0.2) (layer "F.Cu") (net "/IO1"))
 (segment (start 11.8787 19.32) (end 12.2787 18.92) (width 0.2) (layer "F.Cu") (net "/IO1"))
 (segment (start 10.8 19.32) (end 11.8787 19.32) (width 0.2) (layer "F.Cu") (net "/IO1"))
 (segment (start 13.09 19.57) (end 21.5 19.57) (width 0.2) (layer "F.Cu") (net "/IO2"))
 (segment (start 10.8 21.86) (end 13.09 19.57) (width 0.2) (layer "F.Cu") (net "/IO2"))
 (segment (start 14.98 20.22) (end 21.5 20.22) (width 0.2) (layer "F.Cu") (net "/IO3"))
 (segment (start 10.8 24.4) (end 14.98 20.22) (width 0.2) (layer "F.Cu") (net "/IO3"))
 (segment (start 10.8 26.94) (end 16.87 20.87) (width 0.2) (layer "F.Cu") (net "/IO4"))
 (segment (start 16.87 20.87) (end 21.5 20.87) (width 0.2) (layer "F.Cu") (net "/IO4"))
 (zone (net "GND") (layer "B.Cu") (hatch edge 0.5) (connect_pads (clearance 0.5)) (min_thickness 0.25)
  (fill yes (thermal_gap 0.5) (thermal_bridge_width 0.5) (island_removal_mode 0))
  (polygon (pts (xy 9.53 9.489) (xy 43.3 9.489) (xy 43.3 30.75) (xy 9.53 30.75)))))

